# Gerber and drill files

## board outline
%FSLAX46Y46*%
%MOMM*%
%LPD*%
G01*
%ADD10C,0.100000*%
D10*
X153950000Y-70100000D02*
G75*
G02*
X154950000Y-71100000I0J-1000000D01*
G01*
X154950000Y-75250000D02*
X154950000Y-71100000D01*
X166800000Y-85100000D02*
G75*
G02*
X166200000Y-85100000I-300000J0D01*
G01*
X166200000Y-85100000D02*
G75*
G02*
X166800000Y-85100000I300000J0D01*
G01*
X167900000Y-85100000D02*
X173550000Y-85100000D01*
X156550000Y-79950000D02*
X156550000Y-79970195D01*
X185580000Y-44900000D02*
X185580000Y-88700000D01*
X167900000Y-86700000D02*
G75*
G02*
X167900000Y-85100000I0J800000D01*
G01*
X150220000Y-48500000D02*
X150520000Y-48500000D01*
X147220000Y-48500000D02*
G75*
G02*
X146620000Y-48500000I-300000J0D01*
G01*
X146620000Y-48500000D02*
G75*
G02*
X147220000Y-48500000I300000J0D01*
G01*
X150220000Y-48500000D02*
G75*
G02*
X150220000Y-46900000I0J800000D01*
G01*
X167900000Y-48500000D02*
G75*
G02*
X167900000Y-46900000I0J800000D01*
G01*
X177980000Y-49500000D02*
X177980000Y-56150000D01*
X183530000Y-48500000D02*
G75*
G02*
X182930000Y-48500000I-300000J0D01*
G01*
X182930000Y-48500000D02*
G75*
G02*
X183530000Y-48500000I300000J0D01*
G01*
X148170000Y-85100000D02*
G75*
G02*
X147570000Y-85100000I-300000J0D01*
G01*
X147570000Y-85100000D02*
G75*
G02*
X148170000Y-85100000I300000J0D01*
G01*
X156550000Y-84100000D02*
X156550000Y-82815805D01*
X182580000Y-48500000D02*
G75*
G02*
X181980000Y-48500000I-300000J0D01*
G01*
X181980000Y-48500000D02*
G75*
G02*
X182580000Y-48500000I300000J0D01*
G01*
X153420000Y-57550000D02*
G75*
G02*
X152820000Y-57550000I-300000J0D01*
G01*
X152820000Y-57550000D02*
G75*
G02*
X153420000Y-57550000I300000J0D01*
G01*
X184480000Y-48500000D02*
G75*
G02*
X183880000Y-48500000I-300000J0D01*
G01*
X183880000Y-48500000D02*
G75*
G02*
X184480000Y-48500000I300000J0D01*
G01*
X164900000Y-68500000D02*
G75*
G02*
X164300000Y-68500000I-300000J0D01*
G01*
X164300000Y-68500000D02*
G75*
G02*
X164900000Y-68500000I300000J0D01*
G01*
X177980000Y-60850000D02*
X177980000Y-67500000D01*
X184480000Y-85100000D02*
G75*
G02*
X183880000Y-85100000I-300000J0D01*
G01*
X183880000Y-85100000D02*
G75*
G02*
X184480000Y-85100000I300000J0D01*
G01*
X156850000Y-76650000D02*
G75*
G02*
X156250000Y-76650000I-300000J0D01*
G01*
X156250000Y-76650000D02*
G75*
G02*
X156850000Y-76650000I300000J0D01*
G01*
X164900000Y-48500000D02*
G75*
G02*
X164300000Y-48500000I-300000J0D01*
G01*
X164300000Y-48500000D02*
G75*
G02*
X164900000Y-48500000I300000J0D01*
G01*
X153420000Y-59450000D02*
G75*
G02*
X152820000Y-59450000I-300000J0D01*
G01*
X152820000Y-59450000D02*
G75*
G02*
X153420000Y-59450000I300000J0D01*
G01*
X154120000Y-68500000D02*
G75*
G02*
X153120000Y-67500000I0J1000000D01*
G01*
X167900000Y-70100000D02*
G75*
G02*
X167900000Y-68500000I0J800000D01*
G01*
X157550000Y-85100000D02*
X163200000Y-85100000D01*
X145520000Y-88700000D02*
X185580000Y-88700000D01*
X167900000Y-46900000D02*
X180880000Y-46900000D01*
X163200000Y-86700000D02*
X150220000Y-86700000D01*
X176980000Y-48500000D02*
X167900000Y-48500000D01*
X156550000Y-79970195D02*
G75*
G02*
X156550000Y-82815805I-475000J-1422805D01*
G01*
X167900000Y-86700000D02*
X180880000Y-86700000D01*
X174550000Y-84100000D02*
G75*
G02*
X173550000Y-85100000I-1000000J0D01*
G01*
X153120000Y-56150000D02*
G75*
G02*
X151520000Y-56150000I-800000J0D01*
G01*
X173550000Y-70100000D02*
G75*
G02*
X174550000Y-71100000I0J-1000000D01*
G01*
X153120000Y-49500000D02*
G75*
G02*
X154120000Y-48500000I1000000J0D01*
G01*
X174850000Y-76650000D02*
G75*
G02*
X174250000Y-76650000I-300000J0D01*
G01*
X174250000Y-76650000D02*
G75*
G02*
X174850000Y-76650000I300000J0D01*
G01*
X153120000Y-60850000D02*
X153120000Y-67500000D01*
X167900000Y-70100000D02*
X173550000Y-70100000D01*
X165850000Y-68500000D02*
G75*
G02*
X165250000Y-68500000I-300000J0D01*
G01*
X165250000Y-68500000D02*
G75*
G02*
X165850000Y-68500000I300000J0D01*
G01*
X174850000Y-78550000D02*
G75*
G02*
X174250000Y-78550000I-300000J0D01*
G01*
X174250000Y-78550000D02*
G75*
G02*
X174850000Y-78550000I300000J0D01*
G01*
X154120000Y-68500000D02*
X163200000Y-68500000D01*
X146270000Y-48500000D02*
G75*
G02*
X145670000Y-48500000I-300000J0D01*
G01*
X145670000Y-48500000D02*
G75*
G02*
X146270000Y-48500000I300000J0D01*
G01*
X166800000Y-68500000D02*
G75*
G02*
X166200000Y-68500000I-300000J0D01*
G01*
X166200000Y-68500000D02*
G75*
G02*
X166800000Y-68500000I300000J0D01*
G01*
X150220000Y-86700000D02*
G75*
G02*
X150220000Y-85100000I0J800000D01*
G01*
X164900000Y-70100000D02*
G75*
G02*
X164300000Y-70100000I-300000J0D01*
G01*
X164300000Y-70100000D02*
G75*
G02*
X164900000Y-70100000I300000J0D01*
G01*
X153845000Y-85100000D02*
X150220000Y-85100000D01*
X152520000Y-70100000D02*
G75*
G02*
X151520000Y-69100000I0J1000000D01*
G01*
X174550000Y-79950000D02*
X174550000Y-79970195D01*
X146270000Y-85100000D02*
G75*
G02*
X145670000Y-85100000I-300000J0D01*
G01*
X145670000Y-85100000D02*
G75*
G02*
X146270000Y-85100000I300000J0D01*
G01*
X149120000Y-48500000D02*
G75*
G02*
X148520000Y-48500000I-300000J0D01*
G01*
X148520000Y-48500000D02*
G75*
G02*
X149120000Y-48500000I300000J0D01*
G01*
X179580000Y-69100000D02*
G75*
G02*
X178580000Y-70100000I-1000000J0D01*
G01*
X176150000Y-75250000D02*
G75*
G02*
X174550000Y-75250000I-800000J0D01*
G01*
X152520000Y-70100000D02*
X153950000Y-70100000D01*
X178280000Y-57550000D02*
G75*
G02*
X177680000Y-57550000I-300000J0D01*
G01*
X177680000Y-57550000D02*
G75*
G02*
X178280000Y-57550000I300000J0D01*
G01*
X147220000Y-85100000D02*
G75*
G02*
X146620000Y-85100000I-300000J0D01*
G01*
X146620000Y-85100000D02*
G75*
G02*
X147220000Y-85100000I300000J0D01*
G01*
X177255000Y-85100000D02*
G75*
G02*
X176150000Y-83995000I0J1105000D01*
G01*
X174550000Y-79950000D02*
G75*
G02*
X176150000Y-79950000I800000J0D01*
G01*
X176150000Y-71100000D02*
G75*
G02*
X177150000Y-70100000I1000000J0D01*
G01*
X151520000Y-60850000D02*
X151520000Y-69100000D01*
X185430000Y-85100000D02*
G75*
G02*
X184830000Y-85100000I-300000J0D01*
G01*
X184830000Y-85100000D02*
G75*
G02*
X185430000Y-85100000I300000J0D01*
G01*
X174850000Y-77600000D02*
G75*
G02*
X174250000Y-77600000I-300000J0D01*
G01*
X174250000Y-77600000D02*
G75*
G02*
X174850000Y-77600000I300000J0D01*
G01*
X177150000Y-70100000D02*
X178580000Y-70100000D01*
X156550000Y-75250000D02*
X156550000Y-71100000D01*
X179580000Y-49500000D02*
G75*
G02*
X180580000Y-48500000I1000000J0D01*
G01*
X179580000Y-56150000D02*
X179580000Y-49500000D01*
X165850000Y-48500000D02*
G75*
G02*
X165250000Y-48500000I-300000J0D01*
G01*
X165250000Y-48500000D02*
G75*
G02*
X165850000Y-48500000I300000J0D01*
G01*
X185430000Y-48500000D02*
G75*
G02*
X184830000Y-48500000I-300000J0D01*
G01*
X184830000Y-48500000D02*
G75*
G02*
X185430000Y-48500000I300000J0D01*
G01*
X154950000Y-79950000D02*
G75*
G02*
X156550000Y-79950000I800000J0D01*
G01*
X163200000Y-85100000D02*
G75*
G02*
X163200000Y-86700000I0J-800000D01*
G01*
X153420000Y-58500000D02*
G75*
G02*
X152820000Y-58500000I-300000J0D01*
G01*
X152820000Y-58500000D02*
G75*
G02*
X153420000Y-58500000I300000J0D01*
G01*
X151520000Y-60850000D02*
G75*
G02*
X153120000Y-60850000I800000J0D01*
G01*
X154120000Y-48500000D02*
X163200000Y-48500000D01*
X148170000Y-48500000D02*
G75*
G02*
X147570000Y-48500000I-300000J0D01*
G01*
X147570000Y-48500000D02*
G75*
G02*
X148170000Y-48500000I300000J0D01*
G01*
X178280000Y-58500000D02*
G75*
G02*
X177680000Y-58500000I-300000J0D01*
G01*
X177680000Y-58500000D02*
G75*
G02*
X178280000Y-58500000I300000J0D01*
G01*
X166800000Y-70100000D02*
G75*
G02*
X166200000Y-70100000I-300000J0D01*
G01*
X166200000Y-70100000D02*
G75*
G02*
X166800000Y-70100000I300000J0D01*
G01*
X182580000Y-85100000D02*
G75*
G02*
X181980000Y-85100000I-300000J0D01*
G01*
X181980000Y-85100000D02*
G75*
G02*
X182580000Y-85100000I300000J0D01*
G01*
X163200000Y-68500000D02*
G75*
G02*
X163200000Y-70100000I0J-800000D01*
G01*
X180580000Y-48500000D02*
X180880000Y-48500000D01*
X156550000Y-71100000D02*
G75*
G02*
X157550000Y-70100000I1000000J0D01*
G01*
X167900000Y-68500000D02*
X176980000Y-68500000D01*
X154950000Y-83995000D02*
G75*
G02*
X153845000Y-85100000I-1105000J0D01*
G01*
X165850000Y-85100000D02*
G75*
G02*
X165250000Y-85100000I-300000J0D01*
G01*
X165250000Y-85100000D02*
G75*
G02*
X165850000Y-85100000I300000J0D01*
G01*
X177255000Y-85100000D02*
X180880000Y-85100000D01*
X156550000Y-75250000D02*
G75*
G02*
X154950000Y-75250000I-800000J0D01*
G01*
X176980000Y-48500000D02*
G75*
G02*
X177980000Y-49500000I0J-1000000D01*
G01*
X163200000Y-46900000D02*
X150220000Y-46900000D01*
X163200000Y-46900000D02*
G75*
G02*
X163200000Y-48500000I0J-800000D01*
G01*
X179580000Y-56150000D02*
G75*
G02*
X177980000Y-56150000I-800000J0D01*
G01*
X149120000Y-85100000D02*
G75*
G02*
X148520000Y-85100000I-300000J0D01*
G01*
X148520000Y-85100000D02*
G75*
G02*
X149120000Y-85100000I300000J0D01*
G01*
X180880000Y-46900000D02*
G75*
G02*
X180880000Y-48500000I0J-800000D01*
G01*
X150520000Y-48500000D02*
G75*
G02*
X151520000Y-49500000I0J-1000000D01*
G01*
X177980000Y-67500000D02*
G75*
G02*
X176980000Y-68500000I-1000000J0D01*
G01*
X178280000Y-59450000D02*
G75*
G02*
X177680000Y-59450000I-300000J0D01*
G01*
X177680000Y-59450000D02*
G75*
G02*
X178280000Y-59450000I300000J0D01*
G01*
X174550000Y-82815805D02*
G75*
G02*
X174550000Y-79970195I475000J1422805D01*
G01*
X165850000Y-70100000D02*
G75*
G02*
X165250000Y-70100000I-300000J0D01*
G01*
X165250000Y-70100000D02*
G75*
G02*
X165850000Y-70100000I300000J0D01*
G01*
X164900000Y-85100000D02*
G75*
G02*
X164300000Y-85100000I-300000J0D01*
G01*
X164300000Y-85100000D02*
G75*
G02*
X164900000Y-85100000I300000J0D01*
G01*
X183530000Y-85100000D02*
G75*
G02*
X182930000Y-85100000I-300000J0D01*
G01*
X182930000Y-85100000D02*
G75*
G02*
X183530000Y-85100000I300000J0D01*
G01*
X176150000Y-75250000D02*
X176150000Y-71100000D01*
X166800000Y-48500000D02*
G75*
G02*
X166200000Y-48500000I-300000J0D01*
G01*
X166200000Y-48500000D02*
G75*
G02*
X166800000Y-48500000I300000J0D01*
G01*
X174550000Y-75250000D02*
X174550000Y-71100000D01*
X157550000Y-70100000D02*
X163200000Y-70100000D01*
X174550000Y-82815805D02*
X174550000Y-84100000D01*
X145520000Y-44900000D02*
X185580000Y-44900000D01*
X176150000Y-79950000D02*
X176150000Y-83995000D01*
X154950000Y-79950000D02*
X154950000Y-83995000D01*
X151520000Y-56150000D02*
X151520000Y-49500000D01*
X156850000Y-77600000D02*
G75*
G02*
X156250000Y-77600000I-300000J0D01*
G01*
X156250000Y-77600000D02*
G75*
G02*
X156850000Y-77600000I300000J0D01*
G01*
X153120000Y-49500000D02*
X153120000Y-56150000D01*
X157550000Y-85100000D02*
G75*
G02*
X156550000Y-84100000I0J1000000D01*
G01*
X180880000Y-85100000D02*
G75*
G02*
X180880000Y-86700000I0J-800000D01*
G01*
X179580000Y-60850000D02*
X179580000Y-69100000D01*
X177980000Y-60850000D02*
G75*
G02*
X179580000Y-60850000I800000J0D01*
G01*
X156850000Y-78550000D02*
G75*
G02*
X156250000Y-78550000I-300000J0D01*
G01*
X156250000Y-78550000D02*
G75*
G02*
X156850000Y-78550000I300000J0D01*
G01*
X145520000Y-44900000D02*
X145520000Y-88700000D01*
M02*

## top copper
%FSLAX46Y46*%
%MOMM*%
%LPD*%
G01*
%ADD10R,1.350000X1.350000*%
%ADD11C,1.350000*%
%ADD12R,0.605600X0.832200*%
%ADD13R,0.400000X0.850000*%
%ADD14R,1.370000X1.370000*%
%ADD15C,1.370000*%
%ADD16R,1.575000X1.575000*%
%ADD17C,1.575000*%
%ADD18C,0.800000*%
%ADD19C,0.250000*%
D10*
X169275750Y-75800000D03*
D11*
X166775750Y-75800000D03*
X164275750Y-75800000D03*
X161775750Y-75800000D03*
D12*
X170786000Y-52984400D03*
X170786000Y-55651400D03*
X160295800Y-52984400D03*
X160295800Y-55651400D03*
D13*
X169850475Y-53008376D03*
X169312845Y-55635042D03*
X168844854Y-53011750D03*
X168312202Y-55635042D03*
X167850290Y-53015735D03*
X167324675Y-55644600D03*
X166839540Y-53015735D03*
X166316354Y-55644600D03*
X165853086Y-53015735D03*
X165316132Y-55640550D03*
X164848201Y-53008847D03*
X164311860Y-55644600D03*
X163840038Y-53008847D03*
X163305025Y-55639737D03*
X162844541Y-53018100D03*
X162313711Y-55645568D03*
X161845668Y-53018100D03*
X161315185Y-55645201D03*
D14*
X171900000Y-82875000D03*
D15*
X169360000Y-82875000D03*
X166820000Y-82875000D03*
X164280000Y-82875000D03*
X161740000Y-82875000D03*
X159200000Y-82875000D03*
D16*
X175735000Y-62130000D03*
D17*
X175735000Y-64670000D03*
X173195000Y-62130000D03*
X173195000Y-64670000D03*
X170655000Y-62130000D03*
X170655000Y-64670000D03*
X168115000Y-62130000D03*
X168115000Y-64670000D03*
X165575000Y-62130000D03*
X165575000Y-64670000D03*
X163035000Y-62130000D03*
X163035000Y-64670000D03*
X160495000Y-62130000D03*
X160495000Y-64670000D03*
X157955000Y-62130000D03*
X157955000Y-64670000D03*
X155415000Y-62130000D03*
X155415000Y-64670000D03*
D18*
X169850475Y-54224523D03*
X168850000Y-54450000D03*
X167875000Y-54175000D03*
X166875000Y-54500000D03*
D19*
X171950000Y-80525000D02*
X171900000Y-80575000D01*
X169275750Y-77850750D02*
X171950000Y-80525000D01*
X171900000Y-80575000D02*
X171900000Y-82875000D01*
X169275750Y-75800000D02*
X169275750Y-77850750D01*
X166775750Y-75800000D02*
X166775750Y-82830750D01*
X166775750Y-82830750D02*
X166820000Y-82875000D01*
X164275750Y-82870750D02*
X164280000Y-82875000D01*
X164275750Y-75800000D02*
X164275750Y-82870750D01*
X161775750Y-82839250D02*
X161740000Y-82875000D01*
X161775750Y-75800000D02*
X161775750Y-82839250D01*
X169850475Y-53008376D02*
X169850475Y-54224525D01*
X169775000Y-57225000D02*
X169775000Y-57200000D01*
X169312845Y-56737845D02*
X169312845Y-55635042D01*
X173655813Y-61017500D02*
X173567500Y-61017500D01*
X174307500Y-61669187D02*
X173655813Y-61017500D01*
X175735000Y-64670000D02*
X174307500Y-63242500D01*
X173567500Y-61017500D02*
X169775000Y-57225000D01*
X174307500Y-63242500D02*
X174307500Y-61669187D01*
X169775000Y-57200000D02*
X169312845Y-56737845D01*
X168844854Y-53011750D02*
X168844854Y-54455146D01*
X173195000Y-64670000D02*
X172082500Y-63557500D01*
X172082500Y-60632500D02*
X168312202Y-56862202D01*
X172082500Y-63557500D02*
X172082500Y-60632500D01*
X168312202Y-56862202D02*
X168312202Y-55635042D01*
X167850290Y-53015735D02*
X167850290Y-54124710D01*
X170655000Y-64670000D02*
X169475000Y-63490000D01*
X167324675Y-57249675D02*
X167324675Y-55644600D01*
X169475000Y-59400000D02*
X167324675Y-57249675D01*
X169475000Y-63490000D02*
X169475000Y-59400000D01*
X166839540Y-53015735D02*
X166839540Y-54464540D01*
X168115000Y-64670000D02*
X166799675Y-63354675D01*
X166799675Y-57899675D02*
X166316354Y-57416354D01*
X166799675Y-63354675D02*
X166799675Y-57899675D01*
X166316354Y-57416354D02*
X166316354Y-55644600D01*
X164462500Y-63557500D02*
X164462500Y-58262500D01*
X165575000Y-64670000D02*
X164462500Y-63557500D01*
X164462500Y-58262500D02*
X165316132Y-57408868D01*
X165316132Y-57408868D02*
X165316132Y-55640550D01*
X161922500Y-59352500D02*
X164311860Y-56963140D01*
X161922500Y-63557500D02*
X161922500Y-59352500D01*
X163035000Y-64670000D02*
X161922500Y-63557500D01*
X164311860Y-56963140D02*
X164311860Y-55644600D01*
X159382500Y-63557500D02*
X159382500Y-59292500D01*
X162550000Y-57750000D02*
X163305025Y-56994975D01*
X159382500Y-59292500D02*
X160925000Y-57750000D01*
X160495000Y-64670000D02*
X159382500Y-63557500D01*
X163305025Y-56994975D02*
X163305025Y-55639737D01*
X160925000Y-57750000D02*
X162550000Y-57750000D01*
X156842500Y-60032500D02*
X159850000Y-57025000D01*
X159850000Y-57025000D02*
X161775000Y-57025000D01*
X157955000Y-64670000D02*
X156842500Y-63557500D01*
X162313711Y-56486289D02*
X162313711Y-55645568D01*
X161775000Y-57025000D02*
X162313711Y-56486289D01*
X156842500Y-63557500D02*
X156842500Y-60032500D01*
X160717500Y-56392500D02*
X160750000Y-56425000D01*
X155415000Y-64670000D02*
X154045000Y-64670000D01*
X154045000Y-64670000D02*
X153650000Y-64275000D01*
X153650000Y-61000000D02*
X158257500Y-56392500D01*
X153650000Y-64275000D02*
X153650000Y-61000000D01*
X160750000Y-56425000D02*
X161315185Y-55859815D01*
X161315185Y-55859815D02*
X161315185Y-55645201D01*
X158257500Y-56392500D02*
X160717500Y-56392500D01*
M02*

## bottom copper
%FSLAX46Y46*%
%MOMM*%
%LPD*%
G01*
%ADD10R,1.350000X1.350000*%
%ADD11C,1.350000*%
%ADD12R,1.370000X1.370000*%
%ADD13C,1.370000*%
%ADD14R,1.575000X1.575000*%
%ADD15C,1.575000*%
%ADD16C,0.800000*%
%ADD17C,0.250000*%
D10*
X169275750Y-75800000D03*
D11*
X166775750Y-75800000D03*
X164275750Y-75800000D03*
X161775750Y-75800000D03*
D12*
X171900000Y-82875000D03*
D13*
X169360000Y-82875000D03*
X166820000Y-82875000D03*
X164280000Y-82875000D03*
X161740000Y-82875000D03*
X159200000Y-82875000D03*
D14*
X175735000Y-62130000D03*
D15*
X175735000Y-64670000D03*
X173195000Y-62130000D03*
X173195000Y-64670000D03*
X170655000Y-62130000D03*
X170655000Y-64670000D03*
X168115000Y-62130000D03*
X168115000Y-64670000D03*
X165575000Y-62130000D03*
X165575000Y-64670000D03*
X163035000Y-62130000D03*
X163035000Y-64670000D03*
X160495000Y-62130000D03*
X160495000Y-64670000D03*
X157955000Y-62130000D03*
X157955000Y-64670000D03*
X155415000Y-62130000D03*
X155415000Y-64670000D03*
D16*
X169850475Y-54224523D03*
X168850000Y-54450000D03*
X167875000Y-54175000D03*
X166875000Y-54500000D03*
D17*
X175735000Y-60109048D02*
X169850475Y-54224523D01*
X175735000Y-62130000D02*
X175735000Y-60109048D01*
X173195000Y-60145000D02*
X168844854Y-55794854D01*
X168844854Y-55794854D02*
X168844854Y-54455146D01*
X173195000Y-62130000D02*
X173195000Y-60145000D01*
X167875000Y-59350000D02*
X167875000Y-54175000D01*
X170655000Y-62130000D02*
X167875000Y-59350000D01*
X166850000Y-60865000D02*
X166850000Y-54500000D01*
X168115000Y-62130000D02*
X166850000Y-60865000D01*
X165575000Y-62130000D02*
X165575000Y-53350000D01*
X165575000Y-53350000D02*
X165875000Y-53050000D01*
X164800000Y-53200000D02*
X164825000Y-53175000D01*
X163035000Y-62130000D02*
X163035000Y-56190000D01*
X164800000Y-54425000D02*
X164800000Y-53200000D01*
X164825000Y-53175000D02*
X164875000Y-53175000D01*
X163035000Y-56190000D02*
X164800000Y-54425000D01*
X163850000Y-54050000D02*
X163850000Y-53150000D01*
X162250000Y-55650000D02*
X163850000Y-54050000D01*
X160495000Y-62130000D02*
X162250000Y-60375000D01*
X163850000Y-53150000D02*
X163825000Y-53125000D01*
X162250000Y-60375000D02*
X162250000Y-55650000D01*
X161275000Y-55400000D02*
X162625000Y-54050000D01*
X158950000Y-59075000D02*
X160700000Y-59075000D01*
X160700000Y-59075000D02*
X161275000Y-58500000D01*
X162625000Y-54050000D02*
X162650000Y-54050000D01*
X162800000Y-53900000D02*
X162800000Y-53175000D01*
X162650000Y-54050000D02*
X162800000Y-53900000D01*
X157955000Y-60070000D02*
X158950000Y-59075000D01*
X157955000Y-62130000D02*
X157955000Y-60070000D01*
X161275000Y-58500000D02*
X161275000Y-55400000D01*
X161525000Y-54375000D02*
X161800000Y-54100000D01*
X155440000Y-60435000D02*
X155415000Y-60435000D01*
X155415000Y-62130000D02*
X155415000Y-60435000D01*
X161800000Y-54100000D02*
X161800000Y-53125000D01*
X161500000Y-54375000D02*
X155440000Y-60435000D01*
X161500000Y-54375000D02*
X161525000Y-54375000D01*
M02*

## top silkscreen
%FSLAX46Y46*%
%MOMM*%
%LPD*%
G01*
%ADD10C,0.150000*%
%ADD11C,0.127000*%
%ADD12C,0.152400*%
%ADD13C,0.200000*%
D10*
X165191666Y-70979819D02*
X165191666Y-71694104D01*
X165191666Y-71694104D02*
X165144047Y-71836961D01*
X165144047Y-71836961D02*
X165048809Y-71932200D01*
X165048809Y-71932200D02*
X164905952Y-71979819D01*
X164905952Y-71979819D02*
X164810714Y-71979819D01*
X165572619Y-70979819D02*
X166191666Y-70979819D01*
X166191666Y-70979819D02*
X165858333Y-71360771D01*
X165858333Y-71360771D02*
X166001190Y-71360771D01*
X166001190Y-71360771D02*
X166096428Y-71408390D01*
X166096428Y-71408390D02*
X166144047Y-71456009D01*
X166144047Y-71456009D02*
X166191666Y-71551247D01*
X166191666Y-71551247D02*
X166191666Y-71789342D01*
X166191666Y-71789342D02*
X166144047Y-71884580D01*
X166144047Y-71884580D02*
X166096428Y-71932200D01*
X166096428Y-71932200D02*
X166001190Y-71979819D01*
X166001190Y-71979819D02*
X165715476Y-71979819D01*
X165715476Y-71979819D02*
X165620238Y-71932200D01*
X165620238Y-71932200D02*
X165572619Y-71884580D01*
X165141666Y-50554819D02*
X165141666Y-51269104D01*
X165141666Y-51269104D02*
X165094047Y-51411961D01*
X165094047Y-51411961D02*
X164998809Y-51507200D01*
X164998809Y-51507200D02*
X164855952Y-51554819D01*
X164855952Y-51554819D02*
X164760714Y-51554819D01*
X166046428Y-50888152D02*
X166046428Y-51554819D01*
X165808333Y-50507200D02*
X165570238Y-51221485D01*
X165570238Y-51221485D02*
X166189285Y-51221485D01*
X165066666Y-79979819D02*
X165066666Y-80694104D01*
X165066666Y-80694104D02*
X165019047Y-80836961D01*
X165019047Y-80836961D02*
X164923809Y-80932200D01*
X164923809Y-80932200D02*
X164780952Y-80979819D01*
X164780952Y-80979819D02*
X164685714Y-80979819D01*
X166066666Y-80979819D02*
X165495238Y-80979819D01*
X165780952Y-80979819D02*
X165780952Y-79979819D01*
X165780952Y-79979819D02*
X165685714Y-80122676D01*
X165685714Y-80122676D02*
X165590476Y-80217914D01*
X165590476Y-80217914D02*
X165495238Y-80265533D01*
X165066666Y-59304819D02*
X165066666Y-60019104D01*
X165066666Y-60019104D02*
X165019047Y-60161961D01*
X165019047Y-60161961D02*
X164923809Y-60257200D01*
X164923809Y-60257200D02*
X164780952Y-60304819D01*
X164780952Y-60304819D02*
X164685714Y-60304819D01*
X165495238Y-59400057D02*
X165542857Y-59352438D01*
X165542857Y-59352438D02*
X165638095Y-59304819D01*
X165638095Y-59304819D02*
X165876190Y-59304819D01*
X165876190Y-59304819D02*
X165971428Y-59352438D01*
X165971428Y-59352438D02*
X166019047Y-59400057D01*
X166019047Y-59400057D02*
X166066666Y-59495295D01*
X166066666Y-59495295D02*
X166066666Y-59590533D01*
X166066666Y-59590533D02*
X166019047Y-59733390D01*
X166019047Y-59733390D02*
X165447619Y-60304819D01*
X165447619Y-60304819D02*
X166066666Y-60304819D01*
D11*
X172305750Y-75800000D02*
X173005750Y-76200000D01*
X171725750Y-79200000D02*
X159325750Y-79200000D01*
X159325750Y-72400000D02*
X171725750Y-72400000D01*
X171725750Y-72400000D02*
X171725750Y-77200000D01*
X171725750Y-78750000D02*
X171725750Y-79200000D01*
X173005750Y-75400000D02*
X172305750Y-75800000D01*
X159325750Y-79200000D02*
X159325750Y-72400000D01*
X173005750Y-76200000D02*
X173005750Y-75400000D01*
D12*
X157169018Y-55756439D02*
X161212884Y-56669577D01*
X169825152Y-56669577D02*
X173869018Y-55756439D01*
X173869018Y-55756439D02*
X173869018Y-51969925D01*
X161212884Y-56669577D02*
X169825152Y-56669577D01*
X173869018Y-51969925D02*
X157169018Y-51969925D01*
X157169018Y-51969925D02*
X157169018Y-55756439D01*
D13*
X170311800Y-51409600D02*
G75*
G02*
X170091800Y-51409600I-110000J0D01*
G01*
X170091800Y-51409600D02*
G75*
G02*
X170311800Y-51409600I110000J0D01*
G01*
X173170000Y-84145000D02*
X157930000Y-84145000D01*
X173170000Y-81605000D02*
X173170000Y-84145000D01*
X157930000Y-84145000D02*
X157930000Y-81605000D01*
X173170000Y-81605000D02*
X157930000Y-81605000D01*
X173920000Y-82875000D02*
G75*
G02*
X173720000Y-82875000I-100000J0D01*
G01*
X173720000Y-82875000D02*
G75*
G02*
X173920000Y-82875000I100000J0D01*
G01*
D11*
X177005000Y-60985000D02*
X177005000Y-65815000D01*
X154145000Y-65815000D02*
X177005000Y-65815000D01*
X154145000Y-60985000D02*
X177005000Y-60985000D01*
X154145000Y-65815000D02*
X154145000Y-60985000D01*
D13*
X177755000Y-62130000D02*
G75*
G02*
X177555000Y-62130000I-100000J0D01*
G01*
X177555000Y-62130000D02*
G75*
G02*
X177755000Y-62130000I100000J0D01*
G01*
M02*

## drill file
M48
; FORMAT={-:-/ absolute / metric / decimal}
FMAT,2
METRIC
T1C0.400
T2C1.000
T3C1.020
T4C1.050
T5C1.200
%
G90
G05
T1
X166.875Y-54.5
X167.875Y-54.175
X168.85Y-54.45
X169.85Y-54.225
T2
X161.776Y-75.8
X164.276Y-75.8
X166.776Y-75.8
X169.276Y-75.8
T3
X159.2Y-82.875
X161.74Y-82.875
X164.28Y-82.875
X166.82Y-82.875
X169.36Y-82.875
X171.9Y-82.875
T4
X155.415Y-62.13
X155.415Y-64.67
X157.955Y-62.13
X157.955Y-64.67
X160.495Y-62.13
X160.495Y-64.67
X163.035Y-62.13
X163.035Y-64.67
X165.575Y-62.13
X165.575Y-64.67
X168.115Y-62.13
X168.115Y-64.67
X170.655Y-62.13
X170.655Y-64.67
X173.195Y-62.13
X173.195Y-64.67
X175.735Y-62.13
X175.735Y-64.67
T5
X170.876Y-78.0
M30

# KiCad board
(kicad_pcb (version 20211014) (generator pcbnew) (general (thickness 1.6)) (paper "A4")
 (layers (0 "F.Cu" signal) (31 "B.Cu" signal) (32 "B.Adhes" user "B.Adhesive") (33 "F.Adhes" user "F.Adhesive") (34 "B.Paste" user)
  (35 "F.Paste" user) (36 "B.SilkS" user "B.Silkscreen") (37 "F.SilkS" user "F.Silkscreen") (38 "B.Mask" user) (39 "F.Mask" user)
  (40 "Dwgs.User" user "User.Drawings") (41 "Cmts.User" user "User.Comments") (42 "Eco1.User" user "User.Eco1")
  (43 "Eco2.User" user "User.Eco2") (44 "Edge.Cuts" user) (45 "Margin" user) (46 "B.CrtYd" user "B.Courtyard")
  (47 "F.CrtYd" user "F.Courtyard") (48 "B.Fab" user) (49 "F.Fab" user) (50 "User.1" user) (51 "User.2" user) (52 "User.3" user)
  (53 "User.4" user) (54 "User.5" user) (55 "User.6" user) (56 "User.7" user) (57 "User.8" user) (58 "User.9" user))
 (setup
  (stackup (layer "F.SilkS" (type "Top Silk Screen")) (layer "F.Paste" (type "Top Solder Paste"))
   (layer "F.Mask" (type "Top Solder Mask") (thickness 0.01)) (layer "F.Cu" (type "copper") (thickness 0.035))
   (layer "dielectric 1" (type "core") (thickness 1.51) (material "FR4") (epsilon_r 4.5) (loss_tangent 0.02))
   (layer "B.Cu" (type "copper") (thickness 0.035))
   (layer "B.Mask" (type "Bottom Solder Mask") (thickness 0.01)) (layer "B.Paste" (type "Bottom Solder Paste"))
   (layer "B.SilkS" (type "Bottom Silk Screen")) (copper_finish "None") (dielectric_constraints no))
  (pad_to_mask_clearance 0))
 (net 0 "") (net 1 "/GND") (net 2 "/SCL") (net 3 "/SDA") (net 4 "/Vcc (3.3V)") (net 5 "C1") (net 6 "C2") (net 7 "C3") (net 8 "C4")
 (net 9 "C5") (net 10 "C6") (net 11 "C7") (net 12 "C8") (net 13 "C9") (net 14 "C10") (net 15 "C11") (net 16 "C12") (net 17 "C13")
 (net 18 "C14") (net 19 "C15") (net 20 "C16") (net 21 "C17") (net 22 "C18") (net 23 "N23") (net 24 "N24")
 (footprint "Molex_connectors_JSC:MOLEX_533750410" (layer "F.Cu") (at 169.27575 75.8)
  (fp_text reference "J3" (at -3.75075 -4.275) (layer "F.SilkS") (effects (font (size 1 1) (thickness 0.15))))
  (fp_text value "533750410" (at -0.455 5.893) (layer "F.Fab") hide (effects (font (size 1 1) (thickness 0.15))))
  (fp_line (start 3.03 0) (end 3.73 0.4) (layer "F.SilkS") (width 0.127))
  (fp_line (start 2.45 3.4) (end -9.95 3.4) (layer "F.SilkS") (width 0.127))
  (fp_line (start -9.95 -3.4) (end 2.45 -3.4) (layer "F.SilkS") (width 0.127))
  (fp_line (start 2.45 -3.4) (end 2.45 1.4) (layer "F.SilkS") (width 0.127))
  (fp_line (start 2.45 2.95) (end 2.45 3.4) (layer "F.SilkS") (width 0.127))
  (fp_line (start 3.73 -0.4) (end 3.03 0) (layer "F.SilkS") (width 0.127))
  (fp_line (start -9.95 3.4) (end -9.95 -3.4) (layer "F.SilkS") (width 0.127))
  (fp_line (start 3.73 0.4) (end 3.73 -0.4) (layer "F.SilkS") (width 0.127))
  (pad "" np_thru_hole circle (at 1.6 2.2) (size 1.2 1.2) (drill 1.2) (layers *.Cu *.Mask))
  (pad "1" thru_hole rect (at 0 0) (size 1.35 1.35) (drill 1) (layers *.Cu) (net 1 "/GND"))
  (pad "2" thru_hole circle (at -2.5 0) (size 1.35 1.35) (drill 1) (layers *.Cu) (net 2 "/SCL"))
  (pad "3" thru_hole circle (at -5 0) (size 1.35 1.35) (drill 1) (layers *.Cu) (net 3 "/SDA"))
  (pad "4" thru_hole circle (at -7.5 0) (size 1.35 1.35) (drill 1) (layers *.Cu) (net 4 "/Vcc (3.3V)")))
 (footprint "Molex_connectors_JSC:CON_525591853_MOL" (layer "F.Cu") (at 165.325 53.975)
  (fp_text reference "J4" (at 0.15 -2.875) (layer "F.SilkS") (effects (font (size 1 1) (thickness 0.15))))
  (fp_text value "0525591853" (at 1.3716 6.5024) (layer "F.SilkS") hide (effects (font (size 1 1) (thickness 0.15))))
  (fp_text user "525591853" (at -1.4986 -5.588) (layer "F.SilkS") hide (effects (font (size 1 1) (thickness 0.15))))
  (fp_line (start -8.155982 1.781439) (end -4.112116 2.694577) (layer "F.SilkS") (width 0.1524))
  (fp_line (start 4.500152 2.694577) (end 8.544018 1.781439) (layer "F.SilkS") (width 0.1524))
  (fp_line (start 8.544018 1.781439) (end 8.544018 -2.005075) (layer "F.SilkS") (width 0.1524))
  (fp_line (start -4.112116 2.694577) (end 4.500152 2.694577) (layer "F.SilkS") (width 0.1524))
  (fp_line (start 8.544018 -2.005075) (end -8.155982 -2.005075) (layer "F.SilkS") (width 0.1524))
  (fp_line (start -8.155982 -2.005075) (end -8.155982 1.781439) (layer "F.SilkS") (width 0.1524))
  (fp_circle (center 4.8768 -2.5654) (end 4.9868 -2.5654) (layer "F.SilkS") (width 0.2) (fill none))
  (pad " " smd rect (at 5.461 -0.9906) (size 0.6056 0.8322) (layers "F.Cu" "F.Paste" "F.Mask"))
  (pad " " smd rect (at 5.461 1.6764) (size 0.6056 0.8322) (layers "F.Cu" "F.Paste" "F.Mask"))
  (pad " " smd rect (at -5.0292 -0.9906) (size 0.6056 0.8322) (layers "F.Cu" "F.Paste" "F.Mask"))
  (pad " " smd rect (at -5.0292 1.6764) (size 0.6056 0.8322) (layers "F.Cu" "F.Paste" "F.Mask"))
  (pad "1" smd rect (at 4.525475 -0.966624) (size 0.4 0.85) (layers "F.Cu" "F.Paste" "F.Mask") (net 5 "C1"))
  (pad "2" smd rect (at 3.987845 1.660042) (size 0.4 0.85) (layers "F.Cu" "F.Paste" "F.Mask") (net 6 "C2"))
  (pad "3" smd rect (at 3.519854 -0.96325) (size 0.4 0.85) (layers "F.Cu" "F.Paste" "F.Mask") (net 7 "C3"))
  (pad "4" smd rect (at 2.987202 1.660042) (size 0.4 0.85) (layers "F.Cu" "F.Paste" "F.Mask") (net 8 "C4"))
  (pad "5" smd rect (at 2.52529 -0.959265) (size 0.4 0.85) (layers "F.Cu" "F.Paste" "F.Mask") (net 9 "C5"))
  (pad "6" smd rect (at 1.999675 1.6696) (size 0.4 0.85) (layers "F.Cu" "F.Paste" "F.Mask") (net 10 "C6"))
  (pad "7" smd rect (at 1.51454 -0.959265) (size 0.4 0.85) (layers "F.Cu" "F.Paste" "F.Mask") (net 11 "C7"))
  (pad "8" smd rect (at 0.991354 1.6696) (size 0.4 0.85) (layers "F.Cu" "F.Paste" "F.Mask") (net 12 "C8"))
  (pad "9" smd rect (at 0.528086 -0.959265) (size 0.4 0.85) (layers "F.Cu" "F.Paste" "F.Mask") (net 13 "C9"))
  (pad "10" smd rect (at -0.008868 1.66555) (size 0.4 0.85) (layers "F.Cu" "F.Paste" "F.Mask") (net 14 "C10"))
  (pad "11" smd rect (at -0.476799 -0.966153) (size 0.4 0.85) (layers "F.Cu" "F.Paste" "F.Mask") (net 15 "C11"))
  (pad "12" smd rect (at -1.01314 1.6696) (size 0.4 0.85) (layers "F.Cu" "F.Paste" "F.Mask") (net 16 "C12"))
  (pad "13" smd rect (at -1.484962 -0.966153) (size 0.4 0.85) (layers "F.Cu" "F.Paste" "F.Mask") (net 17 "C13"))
  (pad "14" smd rect (at -2.019975 1.664737) (size 0.4 0.85) (layers "F.Cu" "F.Paste" "F.Mask") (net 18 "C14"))
  (pad "15" smd rect (at -2.480459 -0.9569) (size 0.4 0.85) (layers "F.Cu" "F.Paste" "F.Mask") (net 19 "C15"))
  (pad "16" smd rect (at -3.011289 1.670568) (size 0.4 0.85) (layers "F.Cu" "F.Paste" "F.Mask") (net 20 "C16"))
  (pad "17" smd rect (at -3.479332 -0.9569) (size 0.4 0.85) (layers "F.Cu" "F.Paste" "F.Mask") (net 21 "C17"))
  (pad "18" smd rect (at -4.009815 1.670201) (size 0.4 0.85) (layers "F.Cu" "F.Paste" "F.Mask") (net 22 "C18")))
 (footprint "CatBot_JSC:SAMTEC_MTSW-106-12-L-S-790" (layer "F.Cu") (at 165.55 82.875)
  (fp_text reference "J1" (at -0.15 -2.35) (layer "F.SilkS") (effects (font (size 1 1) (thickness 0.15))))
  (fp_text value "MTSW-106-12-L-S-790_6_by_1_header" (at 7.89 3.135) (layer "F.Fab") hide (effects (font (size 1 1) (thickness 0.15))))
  (fp_line (start 7.62 1.27) (end -7.62 1.27) (layer "F.SilkS") (width 0.2))
  (fp_line (start 7.62 -1.27) (end 7.62 1.27) (layer "F.SilkS") (width 0.2))
  (fp_line (start -7.62 1.27) (end -7.62 -1.27) (layer "F.SilkS") (width 0.2))
  (fp_line (start 7.62 -1.27) (end -7.62 -1.27) (layer "F.SilkS") (width 0.2))
  (fp_circle (center 8.27 0) (end 8.37 0) (layer "F.SilkS") (width 0.2) (fill none))
  (pad "01" thru_hole rect (at 6.35 0) (size 1.37 1.37) (drill 1.02) (layers *.Cu *.Mask) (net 1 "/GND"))
  (pad "02" thru_hole circle (at 3.81 0) (size 1.37 1.37) (drill 1.02) (layers *.Cu *.Mask) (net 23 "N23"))
  (pad "03" thru_hole circle (at 1.27 0) (size 1.37 1.37) (drill 1.02) (layers *.Cu *.Mask) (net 2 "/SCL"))
  (pad "04" thru_hole circle (at -1.27 0) (size 1.37 1.37) (drill 1.02) (layers *.Cu *.Mask) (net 3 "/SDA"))
  (pad "05" thru_hole circle (at -3.81 0) (size 1.37 1.37) (drill 1.02) (layers *.Cu *.Mask) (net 4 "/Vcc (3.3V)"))
  (pad "06" thru_hole circle (at -6.35 0) (size 1.37 1.37) (drill 1.02) (layers *.Cu *.Mask) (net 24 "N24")))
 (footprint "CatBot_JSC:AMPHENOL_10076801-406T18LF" (layer "F.Cu") (at 165.575 63.4 180)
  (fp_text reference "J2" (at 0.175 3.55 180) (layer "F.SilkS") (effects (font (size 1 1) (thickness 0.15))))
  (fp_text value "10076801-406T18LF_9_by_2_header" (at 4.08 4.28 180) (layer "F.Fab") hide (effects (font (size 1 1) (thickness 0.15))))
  (fp_line (start -11.43 2.415) (end -11.43 -2.415) (layer "F.SilkS") (width 0.127))
  (fp_line (start 11.43 -2.415) (end -11.43 -2.415) (layer "F.SilkS") (width 0.127))
  (fp_line (start 11.43 2.415) (end -11.43 2.415) (layer "F.SilkS") (width 0.127))
  (fp_line (start 11.43 -2.415) (end 11.43 2.415) (layer "F.SilkS") (width 0.127))
  (fp_circle (center -12.08 1.27) (end -11.98 1.27) (layer "F.SilkS") (width 0.2) (fill none))
  (pad "01" thru_hole rect (at -10.16 1.27 180) (size 1.575 1.575) (drill 1.05) (layers *.Cu *.Mask) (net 5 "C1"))
  (pad "02" thru_hole circle (at -10.16 -1.27 180) (size 1.575 1.575) (drill 1.05) (layers *.Cu *.Mask) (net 6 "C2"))
  (pad "03" thru_hole circle (at -7.62 1.27 180) (size 1.575 1.575) (drill 1.05) (layers *.Cu *.Mask) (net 7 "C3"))
  (pad "04" thru_hole circle (at -7.62 -1.27 180) (size 1.575 1.575) (drill 1.05) (layers *.Cu *.Mask) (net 8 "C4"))
  (pad "05" thru_hole circle (at -5.08 1.27 180) (size 1.575 1.575) (drill 1.05) (layers *.Cu *.Mask) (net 9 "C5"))
  (pad "06" thru_hole circle (at -5.08 -1.27 180) (size 1.575 1.575) (drill 1.05) (layers *.Cu *.Mask) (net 10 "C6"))
  (pad "07" thru_hole circle (at -2.54 1.27 180) (size 1.575 1.575) (drill 1.05) (layers *.Cu *.Mask) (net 11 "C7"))
  (pad "08" thru_hole circle (at -2.54 -1.27 180) (size 1.575 1.575) (drill 1.05) (layers *.Cu *.Mask) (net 12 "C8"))
  (pad "09" thru_hole circle (at 0 1.27 180) (size 1.575 1.575) (drill 1.05) (layers *.Cu *.Mask) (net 13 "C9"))
  (pad "10" thru_hole circle (at 0 -1.27 180) (size 1.575 1.575) (drill 1.05) (layers *.Cu *.Mask) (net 14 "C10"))
  (pad "11" thru_hole circle (at 2.54 1.27 180) (size 1.575 1.575) (drill 1.05) (layers *.Cu *.Mask) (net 15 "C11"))
  (pad "12" thru_hole circle (at 2.54 -1.27 180) (size 1.575 1.575) (drill 1.05) (layers *.Cu *.Mask) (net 16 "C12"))
  (pad "13" thru_hole circle (at 5.08 1.27 180) (size 1.575 1.575) (drill 1.05) (layers *.Cu *.Mask) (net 17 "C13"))
  (pad "14" thru_hole circle (at 5.08 -1.27 180) (size 1.575 1.575) (drill 1.05) (layers *.Cu *.Mask) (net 18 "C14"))
  (pad "15" thru_hole circle (at 7.62 1.27 180) (size 1.575 1.575) (drill 1.05) (layers *.Cu *.Mask) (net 19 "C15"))
  (pad "16" thru_hole circle (at 7.62 -1.27 180) (size 1.575 1.575) (drill 1.05) (layers *.Cu *.Mask) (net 20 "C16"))
  (pad "17" thru_hole circle (at 10.16 1.27 180) (size 1.575 1.575) (drill 1.05) (layers *.Cu *.Mask) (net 21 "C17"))
  (pad "18" thru_hole circle (at 10.16 -1.27 180) (size 1.575 1.575) (drill 1.05) (layers *.Cu *.Mask) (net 22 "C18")))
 (gr_arc (start 153.95 70.1) (mid 154.657107 70.392893) (end 154.95 71.1) (layer "Edge.Cuts") (width 0.1))
 (gr_line (start 154.95 75.25) (end 154.95 71.1) (layer "Edge.Cuts") (width 0.1))
 (gr_circle (center 166.5 85.1) (end 166.8 85.1) (layer "Edge.Cuts") (width 0.1) (fill none))
 (gr_line (start 167.9 85.1) (end 173.55 85.1) (layer "Edge.Cuts") (width 0.1))
 (gr_line (start 156.55 79.95) (end 156.55 79.970195) (layer "Edge.Cuts") (width 0.1))
 (gr_line (start 185.58 44.9) (end 185.58 88.7) (layer "Edge.Cuts") (width 0.1))
 (gr_arc (start 167.9 86.7) (mid 167.1 85.9) (end 167.9 85.1) (layer "Edge.Cuts") (width 0.1))
 (gr_line (start 150.22 48.5) (end 150.52 48.5) (layer "Edge.Cuts") (width 0.1))
 (gr_circle (center 146.92 48.5) (end 147.22 48.5) (layer "Edge.Cuts") (width 0.1) (fill none))
 (gr_arc (start 150.22 48.5) (mid 149.42 47.7) (end 150.22 46.9) (layer "Edge.Cuts") (width 0.1))
 (gr_arc (start 167.9 48.5) (mid 167.1 47.7) (end 167.9 46.9) (layer "Edge.Cuts") (width 0.1))
 (gr_line (start 177.98 49.5) (end 177.98 56.15) (layer "Edge.Cuts") (width 0.1))
 (gr_circle (center 183.23 48.5) (end 183.53 48.5) (layer "Edge.Cuts") (width 0.1) (fill none))
 (gr_circle (center 147.87 85.1) (end 148.17 85.1) (layer "Edge.Cuts") (width 0.1) (fill none))
 (gr_line (start 156.55 84.1) (end 156.55 82.815805) (layer "Edge.Cuts") (width 0.1))
 (gr_circle (center 182.28 48.5) (end 182.58 48.5) (layer "Edge.Cuts") (width 0.1) (fill none))
 (gr_circle (center 153.12 57.55) (end 153.42 57.55) (layer "Edge.Cuts") (width 0.1) (fill none))
 (gr_circle (center 184.18 48.5) (end 184.48 48.5) (layer "Edge.Cuts") (width 0.1) (fill none))
 (gr_circle (center 164.6 68.5) (end 164.9 68.5) (layer "Edge.Cuts") (width 0.1) (fill none))
 (gr_line (start 177.98 60.85) (end 177.98 67.5) (layer "Edge.Cuts") (width 0.1))
 (gr_circle (center 184.18 85.1) (end 184.48 85.1) (layer "Edge.Cuts") (width 0.1) (fill none))
 (gr_circle (center 156.55 76.65) (end 156.85 76.65) (layer "Edge.Cuts") (width 0.1) (fill none))
 (gr_circle (center 164.6 48.5) (end 164.9 48.5) (layer "Edge.Cuts") (width 0.1) (fill none))
 (gr_circle (center 153.12 59.45) (end 153.42 59.45) (layer "Edge.Cuts") (width 0.1) (fill none))
 (gr_arc (start 154.12 68.5) (mid 153.412893 68.207107) (end 153.12 67.5) (layer "Edge.Cuts") (width 0.1))
 (gr_arc (start 167.9 70.1) (mid 167.1 69.3) (end 167.9 68.5) (layer "Edge.Cuts") (width 0.1))
 (gr_line (start 157.55 85.1) (end 163.2 85.1) (layer "Edge.Cuts") (width 0.1))
 (gr_line (start 145.52 88.7) (end 185.58 88.7) (layer "Edge.Cuts") (width 0.1))
 (gr_line (start 167.9 46.9) (end 180.88 46.9) (layer "Edge.Cuts") (width 0.1))
 (gr_line (start 163.2 86.7) (end 150.22 86.7) (layer "Edge.Cuts") (width 0.1))
 (gr_line (start 176.98 48.5) (end 167.9 48.5) (layer "Edge.Cuts") (width 0.1))
 (gr_arc (start 156.55 79.970195) (mid 157.575 81.393) (end 156.55 82.815805) (layer "Edge.Cuts") (width 0.1))
 (gr_line (start 167.9 86.7) (end 180.88 86.7) (layer "Edge.Cuts") (width 0.1))
 (gr_arc (start 174.55 84.1) (mid 174.257107 84.807107) (end 173.55 85.1) (layer "Edge.Cuts") (width 0.1))
 (gr_arc (start 153.12 56.15) (mid 152.32 56.95) (end 151.52 56.15) (layer "Edge.Cuts") (width 0.1))
 (gr_arc (start 173.55 70.1) (mid 174.257107 70.392893) (end 174.55 71.1) (layer "Edge.Cuts") (width 0.1))
 (gr_arc (start 153.12 49.5) (mid 153.412893 48.792893) (end 154.12 48.5) (layer "Edge.Cuts") (width 0.1))
 (gr_circle (center 174.55 76.65) (end 174.85 76.65) (layer "Edge.Cuts") (width 0.1) (fill none))
 (gr_line (start 153.12 60.85) (end 153.12 67.5) (layer "Edge.Cuts") (width 0.1))
 (gr_line (start 167.9 70.1) (end 173.55 70.1) (layer "Edge.Cuts") (width 0.1))
 (gr_circle (center 165.55 68.5) (end 165.85 68.5) (layer "Edge.Cuts") (width 0.1) (fill none))
 (gr_circle (center 174.55 78.55) (end 174.85 78.55) (layer "Edge.Cuts") (width 0.1) (fill none))
 (gr_line (start 154.12 68.5) (end 163.2 68.5) (layer "Edge.Cuts") (width 0.1))
 (gr_circle (center 145.97 48.5) (end 146.27 48.5) (layer "Edge.Cuts") (width 0.1) (fill none))
 (gr_circle (center 166.5 68.5) (end 166.8 68.5) (layer "Edge.Cuts") (width 0.1) (fill none))
 (gr_arc (start 150.22 86.7) (mid 149.42 85.9) (end 150.22 85.1) (layer "Edge.Cuts") (width 0.1))
 (gr_circle (center 164.6 70.1) (end 164.9 70.1) (layer "Edge.Cuts") (width 0.1) (fill none))
 (gr_line (start 153.845 85.1) (end 150.22 85.1) (layer "Edge.Cuts") (width 0.1))
 (gr_arc (start 152.52 70.1) (mid 151.812893 69.807107) (end 151.52 69.1) (layer "Edge.Cuts") (width 0.1))
 (gr_line (start 174.55 79.95) (end 174.55 79.970195) (layer "Edge.Cuts") (width 0.1))
 (gr_circle (center 145.97 85.1) (end 146.27 85.1) (layer "Edge.Cuts") (width 0.1) (fill none))
 (gr_circle (center 148.82 48.5) (end 149.12 48.5) (layer "Edge.Cuts") (width 0.1) (fill none))
 (gr_arc (start 179.58 69.1) (mid 179.287107 69.807107) (end 178.58 70.1) (layer "Edge.Cuts") (width 0.1))
 (gr_arc (start 176.15 75.25) (mid 175.35 76.05) (end 174.55 75.25) (layer "Edge.Cuts") (width 0.1))
 (gr_line (start 152.52 70.1) (end 153.95 70.1) (layer "Edge.Cuts") (width 0.1))
 (gr_circle (center 177.98 57.55) (end 178.28 57.55) (layer "Edge.Cuts") (width 0.1) (fill none))
 (gr_circle (center 146.92 85.1) (end 147.22 85.1) (layer "Edge.Cuts") (width 0.1) (fill none))
 (gr_arc (start 177.255 85.1) (mid 176.473647 84.776353) (end 176.15 83.995) (layer "Edge.Cuts") (width 0.1))
 (gr_arc (start 174.55 79.95) (mid 175.35 79.15) (end 176.15 79.95) (layer "Edge.Cuts") (width 0.1))
 (gr_arc (start 176.15 71.1) (mid 176.442893 70.392893) (end 177.15 70.1) (layer "Edge.Cuts") (width 0.1))
 (gr_line (start 151.52 60.85) (end 151.52 69.1) (layer "Edge.Cuts") (width 0.1))
 (gr_circle (center 185.13 85.1) (end 185.43 85.1) (layer "Edge.Cuts") (width 0.1) (fill none))
 (gr_circle (center 174.55 77.6) (end 174.85 77.6) (layer "Edge.Cuts") (width 0.1) (fill none))
 (gr_line (start 177.15 70.1) (end 178.58 70.1) (layer "Edge.Cuts") (width 0.1))
 (gr_line (start 156.55 75.25) (end 156.55 71.1) (layer "Edge.Cuts") (width 0.1))
 (gr_arc (start 179.58 49.5) (mid 179.872893 48.792893) (end 180.58 48.5) (layer "Edge.Cuts") (width 0.1))
 (gr_line (start 179.58 56.15) (end 179.58 49.5) (layer "Edge.Cuts") (width 0.1))
 (gr_circle (center 165.55 48.5) (end 165.85 48.5) (layer "Edge.Cuts") (width 0.1) (fill none))
 (gr_circle (center 185.13 48.5) (end 185.43 48.5) (layer "Edge.Cuts") (width 0.1) (fill none))
 (gr_arc (start 154.95 79.95) (mid 155.75 79.15) (end 156.55 79.95) (layer "Edge.Cuts") (width 0.1))
 (gr_arc (start 163.2 85.1) (mid 164 85.9) (end 163.2 86.7) (layer "Edge.Cuts") (width 0.1))
 (gr_circle (center 153.12 58.5) (end 153.42 58.5) (layer "Edge.Cuts") (width 0.1) (fill none))
 (gr_arc (start 151.52 60.85) (mid 152.32 60.05) (end 153.12 60.85) (layer "Edge.Cuts") (width 0.1))
 (gr_line (start 154.12 48.5) (end 163.2 48.5) (layer "Edge.Cuts") (width 0.1))
 (gr_circle (center 147.87 48.5) (end 148.17 48.5) (layer "Edge.Cuts") (width 0.1) (fill none))
 (gr_circle (center 177.98 58.5) (end 178.28 58.5) (layer "Edge.Cuts") (width 0.1) (fill none))
 (gr_circle (center 166.5 70.1) (end 166.8 70.1) (layer "Edge.Cuts") (width 0.1) (fill none))
 (gr_circle (center 182.28 85.1) (end 182.58 85.1) (layer "Edge.Cuts") (width 0.1) (fill none))
 (gr_arc (start 163.2 68.5) (mid 164 69.3) (end 163.2 70.1) (layer "Edge.Cuts") (width 0.1))
 (gr_line (start 180.58 48.5) (end 180.88 48.5) (layer "Edge.Cuts") (width 0.1))
 (gr_arc (start 156.55 71.1) (mid 156.842893 70.392893) (end 157.55 70.1) (layer "Edge.Cuts") (width 0.1))
 (gr_line (start 167.9 68.5) (end 176.98 68.5) (layer "Edge.Cuts") (width 0.1))
 (gr_arc (start 154.95 83.995) (mid 154.626353 84.776353) (end 153.845 85.1) (layer "Edge.Cuts") (width 0.1))
 (gr_circle (center 165.55 85.1) (end 165.85 85.1) (layer "Edge.Cuts") (width 0.1) (fill none))
 (gr_line (start 177.255 85.1) (end 180.88 85.1) (layer "Edge.Cuts") (width 0.1))
 (gr_arc (start 156.55 75.25) (mid 155.75 76.05) (end 154.95 75.25) (layer "Edge.Cuts") (width 0.1))
 (gr_arc (start 176.98 48.5) (mid 177.687107 48.792893) (end 177.98 49.5) (layer "Edge.Cuts") (width 0.1))
 (gr_line (start 163.2 46.9) (end 150.22 46.9) (layer "Edge.Cuts") (width 0.1))
 (gr_arc (start 163.2 46.9) (mid 164 47.7) (end 163.2 48.5) (layer "Edge.Cuts") (width 0.1))
 (gr_arc (start 179.58 56.15) (mid 178.78 56.95) (end 177.98 56.15) (layer "Edge.Cuts") (width 0.1))
 (gr_circle (center 148.82 85.1) (end 149.12 85.1) (layer "Edge.Cuts") (width 0.1) (fill none))
 (gr_arc (start 180.88 46.9) (mid 181.68 47.7) (end 180.88 48.5) (layer "Edge.Cuts") (width 0.1))
 (gr_arc (start 150.52 48.5) (mid 151.227107 48.792893) (end 151.52 49.5) (layer "Edge.Cuts") (width 0.1))
 (gr_arc (start 177.98 67.5) (mid 177.687107 68.207107) (end 176.98 68.5) (layer "Edge.Cuts") (width 0.1))
 (gr_circle (center 177.98 59.45) (end 178.28 59.45) (layer "Edge.Cuts") (width 0.1) (fill none))
 (gr_arc (start 174.55 82.815805) (mid 173.525 81.393) (end 174.55 79.970195) (layer "Edge.Cuts") (width 0.1))
 (gr_circle (center 165.55 70.1) (end 165.85 70.1) (layer "Edge.Cuts") (width 0.1) (fill none))
 (gr_circle (center 164.6 85.1) (end 164.9 85.1) (layer "Edge.Cuts") (width 0.1) (fill none))
 (gr_circle (center 183.23 85.1) (end 183.53 85.1) (layer "Edge.Cuts") (width 0.1) (fill none))
 (gr_line (start 176.15 75.25) (end 176.15 71.1) (layer "Edge.Cuts") (width 0.1))
 (gr_circle (center 166.5 48.5) (end 166.8 48.5) (layer "Edge.Cuts") (width 0.1) (fill none))
 (gr_line (start 174.55 75.25) (end 174.55 71.1) (layer "Edge.Cuts") (width 0.1))
 (gr_line (start 157.55 70.1) (end 163.2 70.1) (layer "Edge.Cuts") (width 0.1))
 (gr_line (start 174.55 82.815805) (end 174.55 84.1) (layer "Edge.Cuts") (width 0.1))
 (gr_line (start 145.52 44.9) (end 185.58 44.9) (layer "Edge.Cuts") (width 0.1))
 (gr_line (start 176.15 79.95) (end 176.15 83.995) (layer "Edge.Cuts") (width 0.1))
 (gr_line (start 154.95 79.95) (end 154.95 83.995) (layer "Edge.Cuts") (width 0.1))
 (gr_line (start 151.52 56.15) (end 151.52 49.5) (layer "Edge.Cuts") (width 0.1))
 (gr_circle (center 156.55 77.6) (end 156.85 77.6) (layer "Edge.Cuts") (width 0.1) (fill none))
 (gr_line (start 153.12 49.5) (end 153.12 56.15) (layer "Edge.Cuts") (width 0.1))
 (gr_arc (start 157.55 85.1) (mid 156.842893 84.807107) (end 156.55 84.1) (layer "Edge.Cuts") (width 0.1))
 (gr_arc (start 180.88 85.1) (mid 181.68 85.9) (end 180.88 86.7) (layer "Edge.Cuts") (width 0.1))
 (gr_line (start 179.58 60.85) (end 179.58 69.1) (layer "Edge.Cuts") (width 0.1))
 (gr_arc (start 177.98 60.85) (mid 178.78 60.05) (end 179.58 60.85) (layer "Edge.Cuts") (width 0.1))
 (gr_circle (center 156.55 78.55) (end 156.85 78.55) (layer "Edge.Cuts") (width 0.1) (fill none))
 (gr_line (start 145.52 44.9) (end 145.52 88.7) (layer "Edge.Cuts") (width 0.1))
 (segment (start 171.95 80.525) (end 171.9 80.575) (width 0.25) (layer "F.Cu") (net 1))
 (segment (start 169.27575 77.85075) (end 171.95 80.525) (width 0.25) (layer "F.Cu") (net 1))
 (segment (start 171.9 80.575) (end 171.9 82.875) (width 0.25) (layer "F.Cu") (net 1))
 (segment (start 169.27575 75.8) (end 169.27575 77.85075) (width 0.25) (layer "F.Cu") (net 1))
 (segment (start 166.77575 75.8) (end 166.77575 82.83075) (width 0.25) (layer "F.Cu") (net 2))
 (segment (start 166.77575 82.83075) (end 166.82 82.875) (width 0.25) (layer "F.Cu") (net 2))
 (segment (start 164.27575 82.87075) (end 164.28 82.875) (width 0.25) (layer "F.Cu") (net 3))
 (segment (start 164.27575 75.8) (end 164.27575 82.87075) (width 0.25) (layer "F.Cu") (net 3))
 (segment (start 161.77575 82.83925) (end 161.74 82.875) (width 0.25) (layer "F.Cu") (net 4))
 (segment (start 161.77575 75.8) (end 161.77575 82.83925) (width 0.25) (layer "F.Cu") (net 4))
 (segment (start 169.850475 53.008376) (end 169.850475 54.224525) (width 0.25) (layer "F.Cu") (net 5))
 (via (at 169.850475 54.224523) (size 0.8) (drill 0.4) (layers "F.Cu" "B.Cu") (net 5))
 (segment (start 175.735 60.109048) (end 169.850475 54.224523) (width 0.25) (layer "B.Cu") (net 5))
 (segment (start 175.735 62.13) (end 175.735 60.109048) (width 0.25) (layer "B.Cu") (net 5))
 (segment (start 169.775 57.225) (end 169.775 57.2) (width 0.25) (layer "F.Cu") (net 6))
 (segment (start 169.312845 56.737845) (end 169.312845 55.635042) (width 0.25) (layer "F.Cu") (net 6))
 (segment (start 173.655813 61.0175) (end 173.5675 61.0175) (width 0.25) (layer "F.Cu") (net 6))
 (segment (start 174.3075 61.669187) (end 173.655813 61.0175) (width 0.25) (layer "F.Cu") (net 6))
 (segment (start 175.735 64.67) (end 174.3075 63.2425) (width 0.25) (layer "F.Cu") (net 6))
 (segment (start 173.5675 61.0175) (end 169.775 57.225) (width 0.25) (layer "F.Cu") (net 6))
 (segment (start 174.3075 63.2425) (end 174.3075 61.669187) (width 0.25) (layer "F.Cu") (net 6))
 (segment (start 169.775 57.2) (end 169.312845 56.737845) (width 0.25) (layer "F.Cu") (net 6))
 (segment (start 168.844854 53.01175) (end 168.844854 54.455146) (width 0.25) (layer "F.Cu") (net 7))
 (via (at 168.85 54.45) (size 0.8) (drill 0.4) (layers "F.Cu" "B.Cu") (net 7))
 (segment (start 173.195 60.145) (end 168.844854 55.794854) (width 0.25) (layer "B.Cu") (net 7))
 (segment (start 168.844854 55.794854) (end 168.844854 54.455146) (width 0.25) (layer "B.Cu") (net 7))
 (segment (start 173.195 62.13) (end 173.195 60.145) (width 0.25) (layer "B.Cu") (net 7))
 (segment (start 173.195 64.67) (end 172.0825 63.5575) (width 0.25) (layer "F.Cu") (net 8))
 (segment (start 172.0825 60.6325) (end 168.312202 56.862202) (width 0.25) (layer "F.Cu") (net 8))
 (segment (start 172.0825 63.5575) (end 172.0825 60.6325) (width 0.25) (layer "F.Cu") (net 8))
 (segment (start 168.312202 56.862202) (end 168.312202 55.635042) (width 0.25) (layer "F.Cu") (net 8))
 (segment (start 167.85029 53.015735) (end 167.85029 54.12471) (width 0.25) (layer "F.Cu") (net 9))
 (via (at 167.875 54.175) (size 0.8) (drill 0.4) (layers "F.Cu" "B.Cu") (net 9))
 (segment (start 167.875 59.35) (end 167.875 54.175) (width 0.25) (layer "B.Cu") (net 9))
 (segment (start 170.655 62.13) (end 167.875 59.35) (width 0.25) (layer "B.Cu") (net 9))
 (segment (start 170.655 64.67) (end 169.475 63.49) (width 0.25) (layer "F.Cu") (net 10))
 (segment (start 167.324675 57.249675) (end 167.324675 55.6446) (width 0.25) (layer "F.Cu") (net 10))
 (segment (start 169.475 59.4) (end 167.324675 57.249675) (width 0.25) (layer "F.Cu") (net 10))
 (segment (start 169.475 63.49) (end 169.475 59.4) (width 0.25) (layer "F.Cu") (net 10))
 (segment (start 166.83954 53.015735) (end 166.83954 54.46454) (width 0.25) (layer "F.Cu") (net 11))
 (via (at 166.875 54.5) (size 0.8) (drill 0.4) (layers "F.Cu" "B.Cu") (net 11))
 (segment (start 166.85 60.865) (end 166.85 54.5) (width 0.25) (layer "B.Cu") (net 11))
 (segment (start 168.115 62.13) (end 166.85 60.865) (width 0.25) (layer "B.Cu") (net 11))
 (segment (start 168.115 64.67) (end 166.799675 63.354675) (width 0.25) (layer "F.Cu") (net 12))
 (segment (start 166.799675 57.899675) (end 166.316354 57.416354) (width 0.25) (layer "F.Cu") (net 12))
 (segment (start 166.799675 63.354675) (end 166.799675 57.899675) (width 0.25) (layer "F.Cu") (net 12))
 (segment (start 166.316354 57.416354) (end 166.316354 55.6446) (width 0.25) (layer "F.Cu") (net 12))
 (segment (start 165.575 62.13) (end 165.575 53.35) (width 0.25) (layer "B.Cu") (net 13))
 (segment (start 165.575 53.35) (end 165.875 53.05) (width 0.25) (layer "B.Cu") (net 13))
 (segment (start 164.4625 63.5575) (end 164.4625 58.2625) (width 0.25) (layer "F.Cu") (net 14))
 (segment (start 165.575 64.67) (end 164.4625 63.5575) (width 0.25) (layer "F.Cu") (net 14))
 (segment (start 164.4625 58.2625) (end 165.316132 57.408868) (width 0.25) (layer "F.Cu") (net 14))
 (segment (start 165.316132 57.408868) (end 165.316132 55.64055) (width 0.25) (layer "F.Cu") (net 14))
 (segment (start 164.8 53.2) (end 164.825 53.175) (width 0.25) (layer "B.Cu") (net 15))
 (segment (start 163.035 62.13) (end 163.035 56.19) (width 0.25) (layer "B.Cu") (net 15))
 (segment (start 164.8 54.425) (end 164.8 53.2) (width 0.25) (layer "B.Cu") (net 15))
 (segment (start 164.825 53.175) (end 164.875 53.175) (width 0.25) (layer "B.Cu") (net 15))
 (segment (start 163.035 56.19) (end 164.8 54.425) (width 0.25) (layer "B.Cu") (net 15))
 (segment (start 161.9225 59.3525) (end 164.31186 56.96314) (width 0.25) (layer "F.Cu") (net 16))
 (segment (start 161.9225 63.5575) (end 161.9225 59.3525) (width 0.25) (layer "F.Cu") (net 16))
 (segment (start 163.035 64.67) (end 161.9225 63.5575) (width 0.25) (layer "F.Cu") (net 16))
 (segment (start 164.31186 56.96314) (end 164.31186 55.6446) (width 0.25) (layer "F.Cu") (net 16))
 (segment (start 163.85 54.05) (end 163.85 53.15) (width 0.25) (layer "B.Cu") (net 17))
 (segment (start 162.25 55.65) (end 163.85 54.05) (width 0.25) (layer "B.Cu") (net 17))
 (segment (start 160.495 62.13) (end 162.25 60.375) (width 0.25) (layer "B.Cu") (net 17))
 (segment (start 163.85 53.15) (end 163.825 53.125) (width 0.25) (layer "B.Cu") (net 17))
 (segment (start 162.25 60.375) (end 162.25 55.65) (width 0.25) (layer "B.Cu") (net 17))
 (segment (start 159.3825 63.5575) (end 159.3825 59.2925) (width 0.25) (layer "F.Cu") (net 18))
 (segment (start 162.55 57.75) (end 163.305025 56.994975) (width 0.25) (layer "F.Cu") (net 18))
 (segment (start 159.3825 59.2925) (end 160.925 57.75) (width 0.25) (layer "F.Cu") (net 18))
 (segment (start 160.495 64.67) (end 159.3825 63.5575) (width 0.25) (layer "F.Cu") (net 18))
 (segment (start 163.305025 56.994975) (end 163.305025 55.639737) (width 0.25) (layer "F.Cu") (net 18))
 (segment (start 160.925 57.75) (end 162.55 57.75) (width 0.25) (layer "F.Cu") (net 18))
 (segment (start 161.275 55.4) (end 162.625 54.05) (width 0.25) (layer "B.Cu") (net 19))
 (segment (start 158.95 59.075) (end 160.7 59.075) (width 0.25) (layer "B.Cu") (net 19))
 (segment (start 160.7 59.075) (end 161.275 58.5) (width 0.25) (layer "B.Cu") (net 19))
 (segment (start 162.625 54.05) (end 162.65 54.05) (width 0.25) (layer "B.Cu") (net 19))
 (segment (start 162.8 53.9) (end 162.8 53.175) (width 0.25) (layer "B.Cu") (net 19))
 (segment (start 162.65 54.05) (end 162.8 53.9) (width 0.25) (layer "B.Cu") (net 19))
 (segment (start 157.955 60.07) (end 158.95 59.075) (width 0.25) (layer "B.Cu") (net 19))
 (segment (start 157.955 62.13) (end 157.955 60.07) (width 0.25) (layer "B.Cu") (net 19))
 (segment (start 161.275 58.5) (end 161.275 55.4) (width 0.25) (layer "B.Cu") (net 19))
 (segment (start 156.8425 60.0325) (end 159.85 57.025) (width 0.25) (layer "F.Cu") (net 20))
 (segment (start 159.85 57.025) (end 161.775 57.025) (width 0.25) (layer "F.Cu") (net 20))
 (segment (start 157.955 64.67) (end 156.8425 63.5575) (width 0.25) (layer "F.Cu") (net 20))
 (segment (start 162.313711 56.486289) (end 162.313711 55.645568) (width 0.25) (layer "F.Cu") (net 20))
 (segment (start 161.775 57.025) (end 162.313711 56.486289) (width 0.25) (layer "F.Cu") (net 20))
 (segment (start 156.8425 63.5575) (end 156.8425 60.0325) (width 0.25) (layer "F.Cu") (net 20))
 (segment (start 161.525 54.375) (end 161.8 54.1) (width 0.25) (layer "B.Cu") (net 21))
 (segment (start 155.44 60.435) (end 155.415 60.435) (width 0.25) (layer "B.Cu") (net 21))
 (segment (start 155.415 62.13) (end 155.415 60.435) (width 0.25) (layer "B.Cu") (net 21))
 (segment (start 161.8 54.1) (end 161.8 53.125) (width 0.25) (layer "B.Cu") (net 21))
 (segment (start 161.5 54.375) (end 155.44 60.435) (width 0.25) (layer "B.Cu") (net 21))
 (segment (start 161.5 54.375) (end 161.525 54.375) (width 0.25) (layer "B.Cu") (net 21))
 (segment (start 160.7175 56.3925) (end 160.75 56.425) (width 0.25) (layer "F.Cu") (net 22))
 (segment (start 155.415 64.67) (end 154.045 64.67) (width 0.25) (layer "F.Cu") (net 22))
 (segment (start 154.045 64.67) (end 153.65 64.275) (width 0.25) (layer "F.Cu") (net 22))
 (segment (start 153.65 61) (end 158.2575 56.3925) (width 0.25) (layer "F.Cu") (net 22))
 (segment (start 153.65 64.275) (end 153.65 61) (width 0.25) (layer "F.Cu") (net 22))
 (segment (start 160.75 56.425) (end 161.315185 55.859815) (width 0.25) (layer "F.Cu") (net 22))
 (segment (start 161.315185 55.859815) (end 161.315185 55.645201) (width 0.25) (layer "F.Cu") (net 22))
 (segment (start 158.2575 56.3925) (end 160.7175 56.3925) (width 0.25) (layer "F.Cu") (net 22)))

